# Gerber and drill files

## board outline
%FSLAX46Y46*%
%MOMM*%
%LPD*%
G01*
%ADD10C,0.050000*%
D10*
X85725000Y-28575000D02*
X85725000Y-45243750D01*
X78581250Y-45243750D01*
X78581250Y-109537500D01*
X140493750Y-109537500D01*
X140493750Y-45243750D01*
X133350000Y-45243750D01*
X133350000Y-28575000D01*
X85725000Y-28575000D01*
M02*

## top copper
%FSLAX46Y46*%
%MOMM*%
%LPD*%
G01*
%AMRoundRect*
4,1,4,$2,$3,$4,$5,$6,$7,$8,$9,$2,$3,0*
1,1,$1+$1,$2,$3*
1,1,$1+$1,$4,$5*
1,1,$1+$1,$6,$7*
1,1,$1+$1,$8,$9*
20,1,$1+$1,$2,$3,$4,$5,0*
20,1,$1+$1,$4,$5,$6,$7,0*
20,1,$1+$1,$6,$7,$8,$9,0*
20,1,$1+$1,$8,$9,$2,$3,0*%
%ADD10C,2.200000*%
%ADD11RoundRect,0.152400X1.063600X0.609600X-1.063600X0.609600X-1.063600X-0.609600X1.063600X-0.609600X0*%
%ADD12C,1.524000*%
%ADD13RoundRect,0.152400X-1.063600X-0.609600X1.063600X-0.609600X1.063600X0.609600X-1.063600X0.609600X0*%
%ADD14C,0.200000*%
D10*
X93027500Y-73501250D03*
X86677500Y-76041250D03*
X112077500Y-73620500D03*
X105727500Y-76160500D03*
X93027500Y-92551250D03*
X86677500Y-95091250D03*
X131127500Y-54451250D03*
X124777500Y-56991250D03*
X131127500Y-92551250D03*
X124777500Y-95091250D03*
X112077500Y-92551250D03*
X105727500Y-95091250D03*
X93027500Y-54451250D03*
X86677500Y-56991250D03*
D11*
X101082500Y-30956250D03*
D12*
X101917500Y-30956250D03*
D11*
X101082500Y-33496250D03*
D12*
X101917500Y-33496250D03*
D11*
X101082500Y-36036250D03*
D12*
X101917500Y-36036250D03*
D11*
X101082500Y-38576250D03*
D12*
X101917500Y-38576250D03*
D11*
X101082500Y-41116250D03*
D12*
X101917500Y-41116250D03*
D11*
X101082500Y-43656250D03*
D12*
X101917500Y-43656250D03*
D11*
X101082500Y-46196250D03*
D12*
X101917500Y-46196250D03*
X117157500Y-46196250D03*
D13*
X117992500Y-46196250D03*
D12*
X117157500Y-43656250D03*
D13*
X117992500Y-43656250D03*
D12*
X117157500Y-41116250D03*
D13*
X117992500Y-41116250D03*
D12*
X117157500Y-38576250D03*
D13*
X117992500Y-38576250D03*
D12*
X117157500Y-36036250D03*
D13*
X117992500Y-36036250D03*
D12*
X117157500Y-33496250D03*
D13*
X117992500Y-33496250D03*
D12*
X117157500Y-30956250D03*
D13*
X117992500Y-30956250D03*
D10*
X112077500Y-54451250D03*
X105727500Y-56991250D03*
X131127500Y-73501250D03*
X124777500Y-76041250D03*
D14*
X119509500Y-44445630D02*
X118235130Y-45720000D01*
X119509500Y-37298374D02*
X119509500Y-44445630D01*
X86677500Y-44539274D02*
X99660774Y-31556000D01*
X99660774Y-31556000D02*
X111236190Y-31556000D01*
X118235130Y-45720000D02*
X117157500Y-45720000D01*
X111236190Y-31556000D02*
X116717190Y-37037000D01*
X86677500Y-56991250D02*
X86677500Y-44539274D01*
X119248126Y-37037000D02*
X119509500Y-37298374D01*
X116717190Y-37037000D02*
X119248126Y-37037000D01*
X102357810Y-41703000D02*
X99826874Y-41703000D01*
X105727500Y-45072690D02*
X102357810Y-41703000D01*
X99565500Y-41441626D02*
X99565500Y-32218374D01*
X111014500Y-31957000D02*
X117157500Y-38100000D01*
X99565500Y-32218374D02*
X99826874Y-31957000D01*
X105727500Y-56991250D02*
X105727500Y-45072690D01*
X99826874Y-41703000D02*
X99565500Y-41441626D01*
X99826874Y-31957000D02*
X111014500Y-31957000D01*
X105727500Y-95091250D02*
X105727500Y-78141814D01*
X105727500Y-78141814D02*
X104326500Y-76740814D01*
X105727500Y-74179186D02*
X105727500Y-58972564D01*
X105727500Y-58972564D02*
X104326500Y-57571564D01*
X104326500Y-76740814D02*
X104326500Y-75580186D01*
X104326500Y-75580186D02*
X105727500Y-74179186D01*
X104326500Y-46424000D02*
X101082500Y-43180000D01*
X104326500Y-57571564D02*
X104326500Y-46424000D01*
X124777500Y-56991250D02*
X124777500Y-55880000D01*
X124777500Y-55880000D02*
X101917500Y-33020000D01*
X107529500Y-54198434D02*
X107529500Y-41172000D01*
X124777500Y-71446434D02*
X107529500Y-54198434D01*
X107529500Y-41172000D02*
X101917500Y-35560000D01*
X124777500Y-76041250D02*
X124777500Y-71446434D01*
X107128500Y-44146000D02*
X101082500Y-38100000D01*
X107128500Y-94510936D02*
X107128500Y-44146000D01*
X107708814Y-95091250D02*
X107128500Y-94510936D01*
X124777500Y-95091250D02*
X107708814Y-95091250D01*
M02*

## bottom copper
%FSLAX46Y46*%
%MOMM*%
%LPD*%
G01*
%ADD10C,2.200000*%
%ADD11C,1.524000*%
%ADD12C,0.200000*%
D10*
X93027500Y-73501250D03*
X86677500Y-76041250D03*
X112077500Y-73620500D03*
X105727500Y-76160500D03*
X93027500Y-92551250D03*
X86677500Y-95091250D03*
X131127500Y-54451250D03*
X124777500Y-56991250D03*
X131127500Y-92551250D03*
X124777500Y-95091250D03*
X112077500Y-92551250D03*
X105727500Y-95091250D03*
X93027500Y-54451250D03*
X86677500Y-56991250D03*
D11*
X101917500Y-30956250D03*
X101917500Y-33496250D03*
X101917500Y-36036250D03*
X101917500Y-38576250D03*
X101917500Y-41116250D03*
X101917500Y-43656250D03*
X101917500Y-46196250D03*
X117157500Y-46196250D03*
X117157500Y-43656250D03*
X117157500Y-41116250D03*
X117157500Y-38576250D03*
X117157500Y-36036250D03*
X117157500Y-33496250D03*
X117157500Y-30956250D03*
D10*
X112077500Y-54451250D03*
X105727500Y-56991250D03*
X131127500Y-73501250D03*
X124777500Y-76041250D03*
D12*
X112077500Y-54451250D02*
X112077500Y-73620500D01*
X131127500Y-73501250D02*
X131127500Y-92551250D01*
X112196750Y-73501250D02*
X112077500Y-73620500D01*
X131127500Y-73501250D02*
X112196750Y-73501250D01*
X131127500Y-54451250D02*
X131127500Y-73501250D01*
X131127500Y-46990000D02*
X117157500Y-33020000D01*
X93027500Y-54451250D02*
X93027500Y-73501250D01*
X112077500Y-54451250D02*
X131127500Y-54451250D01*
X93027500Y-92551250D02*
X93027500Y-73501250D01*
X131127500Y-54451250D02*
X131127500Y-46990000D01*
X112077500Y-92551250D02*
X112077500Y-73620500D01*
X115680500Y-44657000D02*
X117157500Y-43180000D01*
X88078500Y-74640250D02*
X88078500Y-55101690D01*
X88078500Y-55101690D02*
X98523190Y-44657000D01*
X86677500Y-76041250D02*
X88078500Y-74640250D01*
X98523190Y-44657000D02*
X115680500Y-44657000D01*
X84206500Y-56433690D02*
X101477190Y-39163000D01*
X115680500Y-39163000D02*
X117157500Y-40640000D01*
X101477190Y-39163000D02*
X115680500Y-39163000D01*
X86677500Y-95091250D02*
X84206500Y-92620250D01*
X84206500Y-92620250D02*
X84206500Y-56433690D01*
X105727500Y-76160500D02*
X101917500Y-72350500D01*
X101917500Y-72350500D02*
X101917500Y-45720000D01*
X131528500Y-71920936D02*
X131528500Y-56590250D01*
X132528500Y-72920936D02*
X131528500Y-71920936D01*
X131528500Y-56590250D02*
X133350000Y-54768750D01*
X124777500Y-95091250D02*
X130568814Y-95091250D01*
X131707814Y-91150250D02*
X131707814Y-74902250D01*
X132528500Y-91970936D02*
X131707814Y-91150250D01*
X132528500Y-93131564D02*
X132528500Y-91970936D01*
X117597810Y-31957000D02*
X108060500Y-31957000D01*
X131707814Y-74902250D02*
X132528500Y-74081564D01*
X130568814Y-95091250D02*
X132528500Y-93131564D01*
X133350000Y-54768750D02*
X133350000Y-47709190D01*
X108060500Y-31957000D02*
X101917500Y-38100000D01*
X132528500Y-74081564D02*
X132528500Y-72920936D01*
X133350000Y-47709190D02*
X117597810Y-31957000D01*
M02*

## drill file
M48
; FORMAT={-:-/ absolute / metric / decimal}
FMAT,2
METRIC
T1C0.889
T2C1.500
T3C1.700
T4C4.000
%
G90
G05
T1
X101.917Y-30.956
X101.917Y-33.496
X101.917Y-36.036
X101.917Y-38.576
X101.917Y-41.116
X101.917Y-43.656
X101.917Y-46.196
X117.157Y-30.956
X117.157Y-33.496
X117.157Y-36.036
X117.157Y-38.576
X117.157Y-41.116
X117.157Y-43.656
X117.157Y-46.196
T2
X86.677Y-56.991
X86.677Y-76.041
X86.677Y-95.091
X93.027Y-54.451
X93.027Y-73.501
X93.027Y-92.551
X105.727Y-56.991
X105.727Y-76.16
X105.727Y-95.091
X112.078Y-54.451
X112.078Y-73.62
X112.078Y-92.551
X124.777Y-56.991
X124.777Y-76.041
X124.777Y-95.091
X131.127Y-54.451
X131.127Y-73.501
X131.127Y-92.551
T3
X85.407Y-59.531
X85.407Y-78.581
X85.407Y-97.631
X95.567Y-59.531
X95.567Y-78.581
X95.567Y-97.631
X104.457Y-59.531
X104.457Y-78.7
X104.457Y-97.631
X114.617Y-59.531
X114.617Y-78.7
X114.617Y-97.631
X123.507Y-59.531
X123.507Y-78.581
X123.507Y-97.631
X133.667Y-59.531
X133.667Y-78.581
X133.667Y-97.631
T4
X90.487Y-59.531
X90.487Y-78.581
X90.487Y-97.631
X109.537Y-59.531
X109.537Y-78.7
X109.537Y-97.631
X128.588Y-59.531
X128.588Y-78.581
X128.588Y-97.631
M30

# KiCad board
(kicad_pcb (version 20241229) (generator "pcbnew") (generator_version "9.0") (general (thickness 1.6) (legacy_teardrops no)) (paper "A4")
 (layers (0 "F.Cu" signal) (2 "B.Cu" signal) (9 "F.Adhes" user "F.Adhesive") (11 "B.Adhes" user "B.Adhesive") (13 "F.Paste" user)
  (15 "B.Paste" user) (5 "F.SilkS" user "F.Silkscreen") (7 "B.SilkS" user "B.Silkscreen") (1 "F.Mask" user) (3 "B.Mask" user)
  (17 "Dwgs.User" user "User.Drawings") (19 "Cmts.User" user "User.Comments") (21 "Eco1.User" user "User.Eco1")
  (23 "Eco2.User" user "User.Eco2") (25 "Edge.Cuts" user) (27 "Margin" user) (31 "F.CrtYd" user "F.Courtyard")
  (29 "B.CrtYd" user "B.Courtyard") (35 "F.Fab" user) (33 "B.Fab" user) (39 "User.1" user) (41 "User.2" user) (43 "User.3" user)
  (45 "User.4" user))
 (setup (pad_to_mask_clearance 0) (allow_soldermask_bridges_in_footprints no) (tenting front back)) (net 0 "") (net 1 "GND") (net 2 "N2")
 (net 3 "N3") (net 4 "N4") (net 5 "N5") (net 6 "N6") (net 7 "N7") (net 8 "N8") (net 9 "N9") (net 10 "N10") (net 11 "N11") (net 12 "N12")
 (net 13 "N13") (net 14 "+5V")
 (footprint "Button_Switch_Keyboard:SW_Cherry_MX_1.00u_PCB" (layer "F.Cu") (at 93.0275 73.50125)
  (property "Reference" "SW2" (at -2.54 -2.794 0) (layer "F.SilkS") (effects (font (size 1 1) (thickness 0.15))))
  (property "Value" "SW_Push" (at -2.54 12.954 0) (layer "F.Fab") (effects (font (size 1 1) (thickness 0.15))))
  (pad "" np_thru_hole circle (at -7.62 5.08) (size 1.7 1.7) (drill 1.7) (layers "*.Cu" "*.Mask"))
  (pad "" np_thru_hole circle (at -2.54 5.08) (size 4 4) (drill 4) (layers "*.Cu" "*.Mask"))
  (pad "" np_thru_hole circle (at 2.54 5.08) (size 1.7 1.7) (drill 1.7) (layers "*.Cu" "*.Mask"))
  (pad "1" thru_hole circle (at 0 0) (size 2.2 2.2) (drill 1.5) (layers "*.Cu" "*.Mask") (remove_unused_layers no) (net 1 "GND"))
  (pad "2" thru_hole circle (at -6.35 2.54) (size 2.2 2.2) (drill 1.5) (layers "*.Cu" "*.Mask") (remove_unused_layers no) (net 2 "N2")))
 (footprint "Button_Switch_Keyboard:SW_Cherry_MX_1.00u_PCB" (layer "F.Cu") (at 112.0775 73.6205)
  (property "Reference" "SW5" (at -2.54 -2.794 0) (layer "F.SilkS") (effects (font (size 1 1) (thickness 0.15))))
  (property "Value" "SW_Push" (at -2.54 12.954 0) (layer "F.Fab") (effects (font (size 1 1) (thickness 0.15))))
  (pad "" np_thru_hole circle (at -7.62 5.08) (size 1.7 1.7) (drill 1.7) (layers "*.Cu" "*.Mask"))
  (pad "" np_thru_hole circle (at -2.54 5.08) (size 4 4) (drill 4) (layers "*.Cu" "*.Mask"))
  (pad "" np_thru_hole circle (at 2.54 5.08) (size 1.7 1.7) (drill 1.7) (layers "*.Cu" "*.Mask"))
  (pad "1" thru_hole circle (at 0 0) (size 2.2 2.2) (drill 1.5) (layers "*.Cu" "*.Mask") (remove_unused_layers no) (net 1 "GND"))
  (pad "2" thru_hole circle (at -6.35 2.54) (size 2.2 2.2) (drill 1.5) (layers "*.Cu" "*.Mask") (remove_unused_layers no) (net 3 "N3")))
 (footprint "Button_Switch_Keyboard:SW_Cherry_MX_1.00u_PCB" (layer "F.Cu") (at 93.0275 92.55125)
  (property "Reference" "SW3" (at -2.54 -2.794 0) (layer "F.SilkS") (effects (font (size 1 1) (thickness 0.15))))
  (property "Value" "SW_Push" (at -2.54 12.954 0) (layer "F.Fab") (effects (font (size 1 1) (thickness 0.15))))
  (pad "" np_thru_hole circle (at -7.62 5.08) (size 1.7 1.7) (drill 1.7) (layers "*.Cu" "*.Mask"))
  (pad "" np_thru_hole circle (at -2.54 5.08) (size 4 4) (drill 4) (layers "*.Cu" "*.Mask"))
  (pad "" np_thru_hole circle (at 2.54 5.08) (size 1.7 1.7) (drill 1.7) (layers "*.Cu" "*.Mask"))
  (pad "1" thru_hole circle (at 0 0) (size 2.2 2.2) (drill 1.5) (layers "*.Cu" "*.Mask") (remove_unused_layers no) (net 1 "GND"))
  (pad "2" thru_hole circle (at -6.35 2.54) (size 2.2 2.2) (drill 1.5) (layers "*.Cu" "*.Mask") (remove_unused_layers no) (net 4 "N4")))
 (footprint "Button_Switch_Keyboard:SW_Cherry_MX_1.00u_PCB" (layer "F.Cu") (at 131.1275 54.45125)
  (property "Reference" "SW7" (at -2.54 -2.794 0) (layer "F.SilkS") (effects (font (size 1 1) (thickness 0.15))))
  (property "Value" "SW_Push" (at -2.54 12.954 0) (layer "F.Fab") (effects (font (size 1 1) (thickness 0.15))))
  (pad "" np_thru_hole circle (at -7.62 5.08) (size 1.7 1.7) (drill 1.7) (layers "*.Cu" "*.Mask"))
  (pad "" np_thru_hole circle (at -2.54 5.08) (size 4 4) (drill 4) (layers "*.Cu" "*.Mask"))
  (pad "" np_thru_hole circle (at 2.54 5.08) (size 1.7 1.7) (drill 1.7) (layers "*.Cu" "*.Mask"))
  (pad "1" thru_hole circle (at 0 0) (size 2.2 2.2) (drill 1.5) (layers "*.Cu" "*.Mask") (remove_unused_layers no) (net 1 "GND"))
  (pad "2" thru_hole circle (at -6.35 2.54) (size 2.2 2.2) (drill 1.5) (layers "*.Cu" "*.Mask") (remove_unused_layers no) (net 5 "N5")))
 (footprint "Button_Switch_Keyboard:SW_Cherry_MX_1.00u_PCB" (layer "F.Cu") (at 131.1275 92.55125)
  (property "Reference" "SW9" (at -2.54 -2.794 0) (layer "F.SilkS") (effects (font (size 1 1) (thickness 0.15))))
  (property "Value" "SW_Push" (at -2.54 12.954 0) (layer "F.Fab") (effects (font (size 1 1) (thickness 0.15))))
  (pad "" np_thru_hole circle (at -7.62 5.08) (size 1.7 1.7) (drill 1.7) (layers "*.Cu" "*.Mask"))
  (pad "" np_thru_hole circle (at -2.54 5.08) (size 4 4) (drill 4) (layers "*.Cu" "*.Mask"))
  (pad "" np_thru_hole circle (at 2.54 5.08) (size 1.7 1.7) (drill 1.7) (layers "*.Cu" "*.Mask"))
  (pad "1" thru_hole circle (at 0 0) (size 2.2 2.2) (drill 1.5) (layers "*.Cu" "*.Mask") (remove_unused_layers no) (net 1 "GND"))
  (pad "2" thru_hole circle (at -6.35 2.54) (size 2.2 2.2) (drill 1.5) (layers "*.Cu" "*.Mask") (remove_unused_layers no) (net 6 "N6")))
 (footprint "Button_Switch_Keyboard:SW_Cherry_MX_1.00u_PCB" (layer "F.Cu") (at 112.0775 92.55125)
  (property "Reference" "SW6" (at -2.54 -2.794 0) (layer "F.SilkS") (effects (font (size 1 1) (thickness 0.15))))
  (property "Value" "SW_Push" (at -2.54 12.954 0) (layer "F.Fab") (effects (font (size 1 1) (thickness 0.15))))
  (pad "" np_thru_hole circle (at -7.62 5.08) (size 1.7 1.7) (drill 1.7) (layers "*.Cu" "*.Mask"))
  (pad "" np_thru_hole circle (at -2.54 5.08) (size 4 4) (drill 4) (layers "*.Cu" "*.Mask"))
  (pad "" np_thru_hole circle (at 2.54 5.08) (size 1.7 1.7) (drill 1.7) (layers "*.Cu" "*.Mask"))
  (pad "1" thru_hole circle (at 0 0) (size 2.2 2.2) (drill 1.5) (layers "*.Cu" "*.Mask") (remove_unused_layers no) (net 1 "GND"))
  (pad "2" thru_hole circle (at -6.35 2.54) (size 2.2 2.2) (drill 1.5) (layers "*.Cu" "*.Mask") (remove_unused_layers no) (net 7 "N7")))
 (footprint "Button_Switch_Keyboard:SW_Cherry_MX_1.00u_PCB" (layer "F.Cu") (at 93.0275 54.45125)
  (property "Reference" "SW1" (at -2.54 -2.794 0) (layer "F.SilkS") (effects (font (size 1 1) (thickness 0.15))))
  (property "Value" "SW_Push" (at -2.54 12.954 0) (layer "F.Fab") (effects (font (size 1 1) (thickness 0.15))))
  (pad "" np_thru_hole circle (at -7.62 5.08) (size 1.7 1.7) (drill 1.7) (layers "*.Cu" "*.Mask"))
  (pad "" np_thru_hole circle (at -2.54 5.08) (size 4 4) (drill 4) (layers "*.Cu" "*.Mask"))
  (pad "" np_thru_hole circle (at 2.54 5.08) (size 1.7 1.7) (drill 1.7) (layers "*.Cu" "*.Mask"))
  (pad "1" thru_hole circle (at 0 0) (size 2.2 2.2) (drill 1.5) (layers "*.Cu" "*.Mask") (remove_unused_layers no) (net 1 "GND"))
  (pad "2" thru_hole circle (at -6.35 2.54) (size 2.2 2.2) (drill 1.5) (layers "*.Cu" "*.Mask") (remove_unused_layers no) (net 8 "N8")))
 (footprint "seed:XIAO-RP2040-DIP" (layer "F.Cu") (at 109.5375 38.57625)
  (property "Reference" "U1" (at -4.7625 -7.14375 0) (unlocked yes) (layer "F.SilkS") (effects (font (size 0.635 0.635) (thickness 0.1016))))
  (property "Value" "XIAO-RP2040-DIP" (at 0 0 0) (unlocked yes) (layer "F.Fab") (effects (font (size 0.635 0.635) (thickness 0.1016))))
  (pad "1" smd roundrect (at -8.455 -7.62 180) (size 2.432 1.524) (layers "F.Cu" "F.Mask") (roundrect_rratio 0.1) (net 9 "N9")
   (thermal_bridge_angle 45))
  (pad "1" thru_hole circle (at -7.62 -7.62 180) (size 1.524 1.524) (drill 0.889) (layers "*.Cu" "*.Mask") (remove_unused_layers no)
   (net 9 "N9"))
  (pad "2" smd roundrect (at -8.455 -5.08 180) (size 2.432 1.524) (layers "F.Cu" "F.Mask") (roundrect_rratio 0.1) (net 5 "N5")
   (thermal_bridge_angle 45))
  (pad "2" thru_hole circle (at -7.62 -5.08 180) (size 1.524 1.524) (drill 0.889) (layers "*.Cu" "*.Mask") (remove_unused_layers no)
   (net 5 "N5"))
  (pad "3" smd roundrect (at -8.455 -2.54 180) (size 2.432 1.524) (layers "F.Cu" "F.Mask") (roundrect_rratio 0.1) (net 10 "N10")
   (thermal_bridge_angle 45))
  (pad "3" thru_hole circle (at -7.62 -2.54 180) (size 1.524 1.524) (drill 0.889) (layers "*.Cu" "*.Mask") (remove_unused_layers no)
   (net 10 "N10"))
  (pad "4" smd roundrect (at -8.455 0 180) (size 2.432 1.524) (layers "F.Cu" "F.Mask") (roundrect_rratio 0.1) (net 6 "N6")
   (thermal_bridge_angle 45))
  (pad "4" thru_hole circle (at -7.62 0 180) (size 1.524 1.524) (drill 0.889) (layers "*.Cu" "*.Mask") (remove_unused_layers no)
   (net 6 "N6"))
  (pad "5" smd roundrect (at -8.455 2.54 180) (size 2.432 1.524) (layers "F.Cu" "F.Mask") (roundrect_rratio 0.1) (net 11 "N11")
   (thermal_bridge_angle 45))
  (pad "5" thru_hole circle (at -7.62 2.54 180) (size 1.524 1.524) (drill 0.889) (layers "*.Cu" "*.Mask") (remove_unused_layers no)
   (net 11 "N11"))
  (pad "6" smd roundrect (at -8.455 5.08 180) (size 2.432 1.524) (layers "F.Cu" "F.Mask") (roundrect_rratio 0.1) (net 7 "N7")
   (thermal_bridge_angle 45))
  (pad "6" thru_hole circle (at -7.62 5.08 180) (size 1.524 1.524) (drill 0.889) (layers "*.Cu" "*.Mask") (remove_unused_layers no)
   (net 7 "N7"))
  (pad "7" smd roundrect (at -8.455 7.62 180) (size 2.432 1.524) (layers "F.Cu" "F.Mask") (roundrect_rratio 0.1) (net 3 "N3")
   (thermal_bridge_angle 45))
  (pad "7" thru_hole circle (at -7.62 7.62 180) (size 1.524 1.524) (drill 0.889) (layers "*.Cu" "*.Mask") (remove_unused_layers no)
   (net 3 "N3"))
  (pad "8" thru_hole circle (at 7.62 7.62) (size 1.524 1.524) (drill 0.889) (layers "*.Cu" "*.Mask") (remove_unused_layers no) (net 8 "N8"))
  (pad "8" smd roundrect (at 8.455 7.62) (size 2.432 1.524) (layers "F.Cu" "F.Mask") (roundrect_rratio 0.1) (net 8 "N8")
   (thermal_bridge_angle 45))
  (pad "9" thru_hole circle (at 7.62 5.08) (size 1.524 1.524) (drill 0.889) (layers "*.Cu" "*.Mask") (remove_unused_layers no) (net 2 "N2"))
  (pad "9" smd roundrect (at 8.455 5.08) (size 2.432 1.524) (layers "F.Cu" "F.Mask") (roundrect_rratio 0.1) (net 2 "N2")
   (thermal_bridge_angle 45))
  (pad "10" thru_hole circle (at 7.62 2.54) (size 1.524 1.524) (drill 0.889) (layers "*.Cu" "*.Mask") (remove_unused_layers no) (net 4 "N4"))
  (pad "10" smd roundrect (at 8.455 2.54) (size 2.432 1.524) (layers "F.Cu" "F.Mask") (roundrect_rratio 0.1) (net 4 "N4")
   (thermal_bridge_angle 45))
  (pad "11" thru_hole circle (at 7.62 0) (size 1.524 1.524) (drill 0.889) (layers "*.Cu" "*.Mask") (remove_unused_layers no) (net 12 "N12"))
  (pad "11" smd roundrect (at 8.455 0) (size 2.432 1.524) (layers "F.Cu" "F.Mask") (roundrect_rratio 0.1) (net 12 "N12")
   (thermal_bridge_angle 45))
  (pad "12" thru_hole circle (at 7.62 -2.54) (size 1.524 1.524) (drill 0.889) (layers "*.Cu" "*.Mask") (remove_unused_layers no)
   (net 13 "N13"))
  (pad "12" smd roundrect (at 8.455 -2.54) (size 2.432 1.524) (layers "F.Cu" "F.Mask") (roundrect_rratio 0.1) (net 13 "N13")
   (thermal_bridge_angle 45))
  (pad "13" thru_hole circle (at 7.62 -5.08) (size 1.524 1.524) (drill 0.889) (layers "*.Cu" "*.Mask") (remove_unused_layers no)
   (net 1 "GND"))
  (pad "13" smd roundrect (at 8.455 -5.08) (size 2.432 1.524) (layers "F.Cu" "F.Mask") (roundrect_rratio 0.1) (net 1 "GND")
   (thermal_bridge_angle 45))
  (pad "14" thru_hole circle (at 7.62 -7.62) (size 1.524 1.524) (drill 0.889) (layers "*.Cu" "*.Mask") (remove_unused_layers no)
   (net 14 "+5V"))
  (pad "14" smd roundrect (at 8.455 -7.62) (size 2.432 1.524) (layers "F.Cu" "F.Mask") (roundrect_rratio 0.1) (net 14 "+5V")
   (thermal_bridge_angle 45)))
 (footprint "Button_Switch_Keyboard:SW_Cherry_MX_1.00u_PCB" (layer "F.Cu") (at 112.0775 54.45125)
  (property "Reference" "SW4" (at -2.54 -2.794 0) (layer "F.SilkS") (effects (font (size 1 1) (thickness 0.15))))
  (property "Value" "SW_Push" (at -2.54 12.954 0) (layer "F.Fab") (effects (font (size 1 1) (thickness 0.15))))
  (pad "" np_thru_hole circle (at -7.62 5.08) (size 1.7 1.7) (drill 1.7) (layers "*.Cu" "*.Mask"))
  (pad "" np_thru_hole circle (at -2.54 5.08) (size 4 4) (drill 4) (layers "*.Cu" "*.Mask"))
  (pad "" np_thru_hole circle (at 2.54 5.08) (size 1.7 1.7) (drill 1.7) (layers "*.Cu" "*.Mask"))
  (pad "1" thru_hole circle (at 0 0) (size 2.2 2.2) (drill 1.5) (layers "*.Cu" "*.Mask") (remove_unused_layers no) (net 1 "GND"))
  (pad "2" thru_hole circle (at -6.35 2.54) (size 2.2 2.2) (drill 1.5) (layers "*.Cu" "*.Mask") (remove_unused_layers no) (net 12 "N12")))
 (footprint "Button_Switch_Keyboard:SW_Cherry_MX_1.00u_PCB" (layer "F.Cu") (at 131.1275 73.50125)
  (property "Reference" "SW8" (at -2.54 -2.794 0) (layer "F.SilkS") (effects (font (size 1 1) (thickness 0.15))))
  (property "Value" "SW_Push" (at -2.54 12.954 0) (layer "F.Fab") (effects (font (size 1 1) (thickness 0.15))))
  (pad "" np_thru_hole circle (at -7.62 5.08) (size 1.7 1.7) (drill 1.7) (layers "*.Cu" "*.Mask"))
  (pad "" np_thru_hole circle (at -2.54 5.08) (size 4 4) (drill 4) (layers "*.Cu" "*.Mask"))
  (pad "" np_thru_hole circle (at 2.54 5.08) (size 1.7 1.7) (drill 1.7) (layers "*.Cu" "*.Mask"))
  (pad "1" thru_hole circle (at 0 0) (size 2.2 2.2) (drill 1.5) (layers "*.Cu" "*.Mask") (remove_unused_layers no) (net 1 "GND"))
  (pad "2" thru_hole circle (at -6.35 2.54) (size 2.2 2.2) (drill 1.5) (layers "*.Cu" "*.Mask") (remove_unused_layers no) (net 10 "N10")))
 (gr_poly
  (pts (xy 85.725 28.575) (xy 85.725 45.24375) (xy 78.58125 45.24375) (xy 78.58125 109.5375) (xy 140.49375 109.5375) (xy 140.49375 45.24375)
   (xy 133.35 45.24375) (xy 133.35 28.575))
  (stroke (width 0.05) (type solid)) (fill no) (layer "Edge.Cuts"))
 (segment (start 112.0775 54.45125) (end 112.0775 73.6205) (width 0.2) (layer "B.Cu") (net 1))
 (segment (start 131.1275 73.50125) (end 131.1275 92.55125) (width 0.2) (layer "B.Cu") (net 1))
 (segment (start 112.19675 73.50125) (end 112.0775 73.6205) (width 0.2) (layer "B.Cu") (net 1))
 (segment (start 131.1275 73.50125) (end 112.19675 73.50125) (width 0.2) (layer "B.Cu") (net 1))
 (segment (start 131.1275 54.45125) (end 131.1275 73.50125) (width 0.2) (layer "B.Cu") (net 1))
 (segment (start 131.1275 46.99) (end 117.1575 33.02) (width 0.2) (layer "B.Cu") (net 1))
 (segment (start 93.0275 54.45125) (end 93.0275 73.50125) (width 0.2) (layer "B.Cu") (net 1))
 (segment (start 112.0775 54.45125) (end 131.1275 54.45125) (width 0.2) (layer "B.Cu") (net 1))
 (segment (start 93.0275 92.55125) (end 93.0275 73.50125) (width 0.2) (layer "B.Cu") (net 1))
 (segment (start 131.1275 54.45125) (end 131.1275 46.99) (width 0.2) (layer "B.Cu") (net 1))
 (segment (start 112.0775 92.55125) (end 112.0775 73.6205) (width 0.2) (layer "B.Cu") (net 1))
 (segment (start 119.5095 44.44563) (end 118.23513 45.72) (width 0.2) (layer "F.Cu") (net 8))
 (segment (start 119.5095 37.298374) (end 119.5095 44.44563) (width 0.2) (layer "F.Cu") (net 8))
 (segment (start 86.6775 44.539274) (end 99.660774 31.556) (width 0.2) (layer "F.Cu") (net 8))
 (segment (start 99.660774 31.556) (end 111.23619 31.556) (width 0.2) (layer "F.Cu") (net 8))
 (segment (start 118.23513 45.72) (end 117.1575 45.72) (width 0.2) (layer "F.Cu") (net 8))
 (segment (start 111.23619 31.556) (end 116.71719 37.037) (width 0.2) (layer "F.Cu") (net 8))
 (segment (start 86.6775 56.99125) (end 86.6775 44.539274) (width 0.2) (layer "F.Cu") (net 8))
 (segment (start 119.248126 37.037) (end 119.5095 37.298374) (width 0.2) (layer "F.Cu") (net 8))
 (segment (start 116.71719 37.037) (end 119.248126 37.037) (width 0.2) (layer "F.Cu") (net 8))
 (segment (start 115.6805 44.657) (end 117.1575 43.18) (width 0.2) (layer "B.Cu") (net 2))
 (segment (start 88.0785 74.64025) (end 88.0785 55.10169) (width 0.2) (layer "B.Cu") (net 2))
 (segment (start 88.0785 55.10169) (end 98.52319 44.657) (width 0.2) (layer "B.Cu") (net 2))
 (segment (start 86.6775 76.04125) (end 88.0785 74.64025) (width 0.2) (layer "B.Cu") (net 2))
 (segment (start 98.52319 44.657) (end 115.6805 44.657) (width 0.2) (layer "B.Cu") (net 2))
 (segment (start 84.2065 56.43369) (end 101.47719 39.163) (width 0.2) (layer "B.Cu") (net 4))
 (segment (start 115.6805 39.163) (end 117.1575 40.64) (width 0.2) (layer "B.Cu") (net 4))
 (segment (start 101.47719 39.163) (end 115.6805 39.163) (width 0.2) (layer "B.Cu") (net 4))
 (segment (start 86.6775 95.09125) (end 84.2065 92.62025) (width 0.2) (layer "B.Cu") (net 4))
 (segment (start 84.2065 92.62025) (end 84.2065 56.43369) (width 0.2) (layer "B.Cu") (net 4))
 (segment (start 102.35781 41.703) (end 99.826874 41.703) (width 0.2) (layer "F.Cu") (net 12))
 (segment (start 105.7275 45.07269) (end 102.35781 41.703) (width 0.2) (layer "F.Cu") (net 12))
 (segment (start 99.5655 41.441626) (end 99.5655 32.218374) (width 0.2) (layer "F.Cu") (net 12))
 (segment (start 111.0145 31.957) (end 117.1575 38.1) (width 0.2) (layer "F.Cu") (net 12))
 (segment (start 99.5655 32.218374) (end 99.826874 31.957) (width 0.2) (layer "F.Cu") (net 12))
 (segment (start 105.7275 56.99125) (end 105.7275 45.07269) (width 0.2) (layer "F.Cu") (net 12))
 (segment (start 99.826874 41.703) (end 99.5655 41.441626) (width 0.2) (layer "F.Cu") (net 12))
 (segment (start 99.826874 31.957) (end 111.0145 31.957) (width 0.2) (layer "F.Cu") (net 12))
 (segment (start 105.7275 76.1605) (end 101.9175 72.3505) (width 0.2) (layer "B.Cu") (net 3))
 (segment (start 101.9175 72.3505) (end 101.9175 45.72) (width 0.2) (layer "B.Cu") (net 3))
 (segment (start 105.7275 95.09125) (end 105.7275 78.141814) (width 0.2) (layer "F.Cu") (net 7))
 (segment (start 105.7275 78.141814) (end 104.3265 76.740814) (width 0.2) (layer "F.Cu") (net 7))
 (segment (start 105.7275 74.179186) (end 105.7275 58.972564) (width 0.2) (layer "F.Cu") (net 7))
 (segment (start 105.7275 58.972564) (end 104.3265 57.571564) (width 0.2) (layer "F.Cu") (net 7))
 (segment (start 104.3265 76.740814) (end 104.3265 75.580186) (width 0.2) (layer "F.Cu") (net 7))
 (segment (start 104.3265 75.580186) (end 105.7275 74.179186) (width 0.2) (layer "F.Cu") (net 7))
 (segment (start 104.3265 46.424) (end 101.0825 43.18) (width 0.2) (layer "F.Cu") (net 7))
 (segment (start 104.3265 57.571564) (end 104.3265 46.424) (width 0.2) (layer "F.Cu") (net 7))
 (segment (start 124.7775 56.99125) (end 124.7775 55.88) (width 0.2) (layer "F.Cu") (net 5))
 (segment (start 124.7775 55.88) (end 101.9175 33.02) (width 0.2) (layer "F.Cu") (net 5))
 (segment (start 107.5295 54.198434) (end 107.5295 41.172) (width 0.2) (layer "F.Cu") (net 10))
 (segment (start 124.7775 71.446434) (end 107.5295 54.198434) (width 0.2) (layer "F.Cu") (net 10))
 (segment (start 107.5295 41.172) (end 101.9175 35.56) (width 0.2) (layer "F.Cu") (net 10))
 (segment (start 124.7775 76.04125) (end 124.7775 71.446434) (width 0.2) (layer "F.Cu") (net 10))
 (segment (start 107.1285 44.146) (end 101.0825 38.1) (width 0.2) (layer "F.Cu") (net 6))
 (segment (start 107.1285 94.510936) (end 107.1285 44.146) (width 0.2) (layer "F.Cu") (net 6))
 (segment (start 107.708814 95.09125) (end 107.1285 94.510936) (width 0.2) (layer "F.Cu") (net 6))
 (segment (start 124.7775 95.09125) (end 107.708814 95.09125) (width 0.2) (layer "F.Cu") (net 6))
 (segment (start 131.5285 71.920936) (end 131.5285 56.59025) (width 0.2) (layer "B.Cu") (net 6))
 (segment (start 132.5285 72.920936) (end 131.5285 71.920936) (width 0.2) (layer "B.Cu") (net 6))
 (segment (start 131.5285 56.59025) (end 133.35 54.76875) (width 0.2) (layer "B.Cu") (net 6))
 (segment (start 124.7775 95.09125) (end 130.568814 95.09125) (width 0.2) (layer "B.Cu") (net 6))
 (segment (start 131.707814 91.15025) (end 131.707814 74.90225) (width 0.2) (layer "B.Cu") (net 6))
 (segment (start 132.5285 91.970936) (end 131.707814 91.15025) (width 0.2) (layer "B.Cu") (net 6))
 (segment (start 132.5285 93.131564) (end 132.5285 91.970936) (width 0.2) (layer "B.Cu") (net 6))
 (segment (start 117.59781 31.957) (end 108.0605 31.957) (width 0.2) (layer "B.Cu") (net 6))
 (segment (start 131.707814 74.90225) (end 132.5285 74.081564) (width 0.2) (layer "B.Cu") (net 6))
 (segment (start 130.568814 95.09125) (end 132.5285 93.131564) (width 0.2) (layer "B.Cu") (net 6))
 (segment (start 133.35 54.76875) (end 133.35 47.70919) (width 0.2) (layer "B.Cu") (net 6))
 (segment (start 108.0605 31.957) (end 101.9175 38.1) (width 0.2) (layer "B.Cu") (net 6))
 (segment (start 132.5285 74.081564) (end 132.5285 72.920936) (width 0.2) (layer "B.Cu") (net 6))
 (segment (start 133.35 47.70919) (end 117.59781 31.957) (width 0.2) (layer "B.Cu") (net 6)))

